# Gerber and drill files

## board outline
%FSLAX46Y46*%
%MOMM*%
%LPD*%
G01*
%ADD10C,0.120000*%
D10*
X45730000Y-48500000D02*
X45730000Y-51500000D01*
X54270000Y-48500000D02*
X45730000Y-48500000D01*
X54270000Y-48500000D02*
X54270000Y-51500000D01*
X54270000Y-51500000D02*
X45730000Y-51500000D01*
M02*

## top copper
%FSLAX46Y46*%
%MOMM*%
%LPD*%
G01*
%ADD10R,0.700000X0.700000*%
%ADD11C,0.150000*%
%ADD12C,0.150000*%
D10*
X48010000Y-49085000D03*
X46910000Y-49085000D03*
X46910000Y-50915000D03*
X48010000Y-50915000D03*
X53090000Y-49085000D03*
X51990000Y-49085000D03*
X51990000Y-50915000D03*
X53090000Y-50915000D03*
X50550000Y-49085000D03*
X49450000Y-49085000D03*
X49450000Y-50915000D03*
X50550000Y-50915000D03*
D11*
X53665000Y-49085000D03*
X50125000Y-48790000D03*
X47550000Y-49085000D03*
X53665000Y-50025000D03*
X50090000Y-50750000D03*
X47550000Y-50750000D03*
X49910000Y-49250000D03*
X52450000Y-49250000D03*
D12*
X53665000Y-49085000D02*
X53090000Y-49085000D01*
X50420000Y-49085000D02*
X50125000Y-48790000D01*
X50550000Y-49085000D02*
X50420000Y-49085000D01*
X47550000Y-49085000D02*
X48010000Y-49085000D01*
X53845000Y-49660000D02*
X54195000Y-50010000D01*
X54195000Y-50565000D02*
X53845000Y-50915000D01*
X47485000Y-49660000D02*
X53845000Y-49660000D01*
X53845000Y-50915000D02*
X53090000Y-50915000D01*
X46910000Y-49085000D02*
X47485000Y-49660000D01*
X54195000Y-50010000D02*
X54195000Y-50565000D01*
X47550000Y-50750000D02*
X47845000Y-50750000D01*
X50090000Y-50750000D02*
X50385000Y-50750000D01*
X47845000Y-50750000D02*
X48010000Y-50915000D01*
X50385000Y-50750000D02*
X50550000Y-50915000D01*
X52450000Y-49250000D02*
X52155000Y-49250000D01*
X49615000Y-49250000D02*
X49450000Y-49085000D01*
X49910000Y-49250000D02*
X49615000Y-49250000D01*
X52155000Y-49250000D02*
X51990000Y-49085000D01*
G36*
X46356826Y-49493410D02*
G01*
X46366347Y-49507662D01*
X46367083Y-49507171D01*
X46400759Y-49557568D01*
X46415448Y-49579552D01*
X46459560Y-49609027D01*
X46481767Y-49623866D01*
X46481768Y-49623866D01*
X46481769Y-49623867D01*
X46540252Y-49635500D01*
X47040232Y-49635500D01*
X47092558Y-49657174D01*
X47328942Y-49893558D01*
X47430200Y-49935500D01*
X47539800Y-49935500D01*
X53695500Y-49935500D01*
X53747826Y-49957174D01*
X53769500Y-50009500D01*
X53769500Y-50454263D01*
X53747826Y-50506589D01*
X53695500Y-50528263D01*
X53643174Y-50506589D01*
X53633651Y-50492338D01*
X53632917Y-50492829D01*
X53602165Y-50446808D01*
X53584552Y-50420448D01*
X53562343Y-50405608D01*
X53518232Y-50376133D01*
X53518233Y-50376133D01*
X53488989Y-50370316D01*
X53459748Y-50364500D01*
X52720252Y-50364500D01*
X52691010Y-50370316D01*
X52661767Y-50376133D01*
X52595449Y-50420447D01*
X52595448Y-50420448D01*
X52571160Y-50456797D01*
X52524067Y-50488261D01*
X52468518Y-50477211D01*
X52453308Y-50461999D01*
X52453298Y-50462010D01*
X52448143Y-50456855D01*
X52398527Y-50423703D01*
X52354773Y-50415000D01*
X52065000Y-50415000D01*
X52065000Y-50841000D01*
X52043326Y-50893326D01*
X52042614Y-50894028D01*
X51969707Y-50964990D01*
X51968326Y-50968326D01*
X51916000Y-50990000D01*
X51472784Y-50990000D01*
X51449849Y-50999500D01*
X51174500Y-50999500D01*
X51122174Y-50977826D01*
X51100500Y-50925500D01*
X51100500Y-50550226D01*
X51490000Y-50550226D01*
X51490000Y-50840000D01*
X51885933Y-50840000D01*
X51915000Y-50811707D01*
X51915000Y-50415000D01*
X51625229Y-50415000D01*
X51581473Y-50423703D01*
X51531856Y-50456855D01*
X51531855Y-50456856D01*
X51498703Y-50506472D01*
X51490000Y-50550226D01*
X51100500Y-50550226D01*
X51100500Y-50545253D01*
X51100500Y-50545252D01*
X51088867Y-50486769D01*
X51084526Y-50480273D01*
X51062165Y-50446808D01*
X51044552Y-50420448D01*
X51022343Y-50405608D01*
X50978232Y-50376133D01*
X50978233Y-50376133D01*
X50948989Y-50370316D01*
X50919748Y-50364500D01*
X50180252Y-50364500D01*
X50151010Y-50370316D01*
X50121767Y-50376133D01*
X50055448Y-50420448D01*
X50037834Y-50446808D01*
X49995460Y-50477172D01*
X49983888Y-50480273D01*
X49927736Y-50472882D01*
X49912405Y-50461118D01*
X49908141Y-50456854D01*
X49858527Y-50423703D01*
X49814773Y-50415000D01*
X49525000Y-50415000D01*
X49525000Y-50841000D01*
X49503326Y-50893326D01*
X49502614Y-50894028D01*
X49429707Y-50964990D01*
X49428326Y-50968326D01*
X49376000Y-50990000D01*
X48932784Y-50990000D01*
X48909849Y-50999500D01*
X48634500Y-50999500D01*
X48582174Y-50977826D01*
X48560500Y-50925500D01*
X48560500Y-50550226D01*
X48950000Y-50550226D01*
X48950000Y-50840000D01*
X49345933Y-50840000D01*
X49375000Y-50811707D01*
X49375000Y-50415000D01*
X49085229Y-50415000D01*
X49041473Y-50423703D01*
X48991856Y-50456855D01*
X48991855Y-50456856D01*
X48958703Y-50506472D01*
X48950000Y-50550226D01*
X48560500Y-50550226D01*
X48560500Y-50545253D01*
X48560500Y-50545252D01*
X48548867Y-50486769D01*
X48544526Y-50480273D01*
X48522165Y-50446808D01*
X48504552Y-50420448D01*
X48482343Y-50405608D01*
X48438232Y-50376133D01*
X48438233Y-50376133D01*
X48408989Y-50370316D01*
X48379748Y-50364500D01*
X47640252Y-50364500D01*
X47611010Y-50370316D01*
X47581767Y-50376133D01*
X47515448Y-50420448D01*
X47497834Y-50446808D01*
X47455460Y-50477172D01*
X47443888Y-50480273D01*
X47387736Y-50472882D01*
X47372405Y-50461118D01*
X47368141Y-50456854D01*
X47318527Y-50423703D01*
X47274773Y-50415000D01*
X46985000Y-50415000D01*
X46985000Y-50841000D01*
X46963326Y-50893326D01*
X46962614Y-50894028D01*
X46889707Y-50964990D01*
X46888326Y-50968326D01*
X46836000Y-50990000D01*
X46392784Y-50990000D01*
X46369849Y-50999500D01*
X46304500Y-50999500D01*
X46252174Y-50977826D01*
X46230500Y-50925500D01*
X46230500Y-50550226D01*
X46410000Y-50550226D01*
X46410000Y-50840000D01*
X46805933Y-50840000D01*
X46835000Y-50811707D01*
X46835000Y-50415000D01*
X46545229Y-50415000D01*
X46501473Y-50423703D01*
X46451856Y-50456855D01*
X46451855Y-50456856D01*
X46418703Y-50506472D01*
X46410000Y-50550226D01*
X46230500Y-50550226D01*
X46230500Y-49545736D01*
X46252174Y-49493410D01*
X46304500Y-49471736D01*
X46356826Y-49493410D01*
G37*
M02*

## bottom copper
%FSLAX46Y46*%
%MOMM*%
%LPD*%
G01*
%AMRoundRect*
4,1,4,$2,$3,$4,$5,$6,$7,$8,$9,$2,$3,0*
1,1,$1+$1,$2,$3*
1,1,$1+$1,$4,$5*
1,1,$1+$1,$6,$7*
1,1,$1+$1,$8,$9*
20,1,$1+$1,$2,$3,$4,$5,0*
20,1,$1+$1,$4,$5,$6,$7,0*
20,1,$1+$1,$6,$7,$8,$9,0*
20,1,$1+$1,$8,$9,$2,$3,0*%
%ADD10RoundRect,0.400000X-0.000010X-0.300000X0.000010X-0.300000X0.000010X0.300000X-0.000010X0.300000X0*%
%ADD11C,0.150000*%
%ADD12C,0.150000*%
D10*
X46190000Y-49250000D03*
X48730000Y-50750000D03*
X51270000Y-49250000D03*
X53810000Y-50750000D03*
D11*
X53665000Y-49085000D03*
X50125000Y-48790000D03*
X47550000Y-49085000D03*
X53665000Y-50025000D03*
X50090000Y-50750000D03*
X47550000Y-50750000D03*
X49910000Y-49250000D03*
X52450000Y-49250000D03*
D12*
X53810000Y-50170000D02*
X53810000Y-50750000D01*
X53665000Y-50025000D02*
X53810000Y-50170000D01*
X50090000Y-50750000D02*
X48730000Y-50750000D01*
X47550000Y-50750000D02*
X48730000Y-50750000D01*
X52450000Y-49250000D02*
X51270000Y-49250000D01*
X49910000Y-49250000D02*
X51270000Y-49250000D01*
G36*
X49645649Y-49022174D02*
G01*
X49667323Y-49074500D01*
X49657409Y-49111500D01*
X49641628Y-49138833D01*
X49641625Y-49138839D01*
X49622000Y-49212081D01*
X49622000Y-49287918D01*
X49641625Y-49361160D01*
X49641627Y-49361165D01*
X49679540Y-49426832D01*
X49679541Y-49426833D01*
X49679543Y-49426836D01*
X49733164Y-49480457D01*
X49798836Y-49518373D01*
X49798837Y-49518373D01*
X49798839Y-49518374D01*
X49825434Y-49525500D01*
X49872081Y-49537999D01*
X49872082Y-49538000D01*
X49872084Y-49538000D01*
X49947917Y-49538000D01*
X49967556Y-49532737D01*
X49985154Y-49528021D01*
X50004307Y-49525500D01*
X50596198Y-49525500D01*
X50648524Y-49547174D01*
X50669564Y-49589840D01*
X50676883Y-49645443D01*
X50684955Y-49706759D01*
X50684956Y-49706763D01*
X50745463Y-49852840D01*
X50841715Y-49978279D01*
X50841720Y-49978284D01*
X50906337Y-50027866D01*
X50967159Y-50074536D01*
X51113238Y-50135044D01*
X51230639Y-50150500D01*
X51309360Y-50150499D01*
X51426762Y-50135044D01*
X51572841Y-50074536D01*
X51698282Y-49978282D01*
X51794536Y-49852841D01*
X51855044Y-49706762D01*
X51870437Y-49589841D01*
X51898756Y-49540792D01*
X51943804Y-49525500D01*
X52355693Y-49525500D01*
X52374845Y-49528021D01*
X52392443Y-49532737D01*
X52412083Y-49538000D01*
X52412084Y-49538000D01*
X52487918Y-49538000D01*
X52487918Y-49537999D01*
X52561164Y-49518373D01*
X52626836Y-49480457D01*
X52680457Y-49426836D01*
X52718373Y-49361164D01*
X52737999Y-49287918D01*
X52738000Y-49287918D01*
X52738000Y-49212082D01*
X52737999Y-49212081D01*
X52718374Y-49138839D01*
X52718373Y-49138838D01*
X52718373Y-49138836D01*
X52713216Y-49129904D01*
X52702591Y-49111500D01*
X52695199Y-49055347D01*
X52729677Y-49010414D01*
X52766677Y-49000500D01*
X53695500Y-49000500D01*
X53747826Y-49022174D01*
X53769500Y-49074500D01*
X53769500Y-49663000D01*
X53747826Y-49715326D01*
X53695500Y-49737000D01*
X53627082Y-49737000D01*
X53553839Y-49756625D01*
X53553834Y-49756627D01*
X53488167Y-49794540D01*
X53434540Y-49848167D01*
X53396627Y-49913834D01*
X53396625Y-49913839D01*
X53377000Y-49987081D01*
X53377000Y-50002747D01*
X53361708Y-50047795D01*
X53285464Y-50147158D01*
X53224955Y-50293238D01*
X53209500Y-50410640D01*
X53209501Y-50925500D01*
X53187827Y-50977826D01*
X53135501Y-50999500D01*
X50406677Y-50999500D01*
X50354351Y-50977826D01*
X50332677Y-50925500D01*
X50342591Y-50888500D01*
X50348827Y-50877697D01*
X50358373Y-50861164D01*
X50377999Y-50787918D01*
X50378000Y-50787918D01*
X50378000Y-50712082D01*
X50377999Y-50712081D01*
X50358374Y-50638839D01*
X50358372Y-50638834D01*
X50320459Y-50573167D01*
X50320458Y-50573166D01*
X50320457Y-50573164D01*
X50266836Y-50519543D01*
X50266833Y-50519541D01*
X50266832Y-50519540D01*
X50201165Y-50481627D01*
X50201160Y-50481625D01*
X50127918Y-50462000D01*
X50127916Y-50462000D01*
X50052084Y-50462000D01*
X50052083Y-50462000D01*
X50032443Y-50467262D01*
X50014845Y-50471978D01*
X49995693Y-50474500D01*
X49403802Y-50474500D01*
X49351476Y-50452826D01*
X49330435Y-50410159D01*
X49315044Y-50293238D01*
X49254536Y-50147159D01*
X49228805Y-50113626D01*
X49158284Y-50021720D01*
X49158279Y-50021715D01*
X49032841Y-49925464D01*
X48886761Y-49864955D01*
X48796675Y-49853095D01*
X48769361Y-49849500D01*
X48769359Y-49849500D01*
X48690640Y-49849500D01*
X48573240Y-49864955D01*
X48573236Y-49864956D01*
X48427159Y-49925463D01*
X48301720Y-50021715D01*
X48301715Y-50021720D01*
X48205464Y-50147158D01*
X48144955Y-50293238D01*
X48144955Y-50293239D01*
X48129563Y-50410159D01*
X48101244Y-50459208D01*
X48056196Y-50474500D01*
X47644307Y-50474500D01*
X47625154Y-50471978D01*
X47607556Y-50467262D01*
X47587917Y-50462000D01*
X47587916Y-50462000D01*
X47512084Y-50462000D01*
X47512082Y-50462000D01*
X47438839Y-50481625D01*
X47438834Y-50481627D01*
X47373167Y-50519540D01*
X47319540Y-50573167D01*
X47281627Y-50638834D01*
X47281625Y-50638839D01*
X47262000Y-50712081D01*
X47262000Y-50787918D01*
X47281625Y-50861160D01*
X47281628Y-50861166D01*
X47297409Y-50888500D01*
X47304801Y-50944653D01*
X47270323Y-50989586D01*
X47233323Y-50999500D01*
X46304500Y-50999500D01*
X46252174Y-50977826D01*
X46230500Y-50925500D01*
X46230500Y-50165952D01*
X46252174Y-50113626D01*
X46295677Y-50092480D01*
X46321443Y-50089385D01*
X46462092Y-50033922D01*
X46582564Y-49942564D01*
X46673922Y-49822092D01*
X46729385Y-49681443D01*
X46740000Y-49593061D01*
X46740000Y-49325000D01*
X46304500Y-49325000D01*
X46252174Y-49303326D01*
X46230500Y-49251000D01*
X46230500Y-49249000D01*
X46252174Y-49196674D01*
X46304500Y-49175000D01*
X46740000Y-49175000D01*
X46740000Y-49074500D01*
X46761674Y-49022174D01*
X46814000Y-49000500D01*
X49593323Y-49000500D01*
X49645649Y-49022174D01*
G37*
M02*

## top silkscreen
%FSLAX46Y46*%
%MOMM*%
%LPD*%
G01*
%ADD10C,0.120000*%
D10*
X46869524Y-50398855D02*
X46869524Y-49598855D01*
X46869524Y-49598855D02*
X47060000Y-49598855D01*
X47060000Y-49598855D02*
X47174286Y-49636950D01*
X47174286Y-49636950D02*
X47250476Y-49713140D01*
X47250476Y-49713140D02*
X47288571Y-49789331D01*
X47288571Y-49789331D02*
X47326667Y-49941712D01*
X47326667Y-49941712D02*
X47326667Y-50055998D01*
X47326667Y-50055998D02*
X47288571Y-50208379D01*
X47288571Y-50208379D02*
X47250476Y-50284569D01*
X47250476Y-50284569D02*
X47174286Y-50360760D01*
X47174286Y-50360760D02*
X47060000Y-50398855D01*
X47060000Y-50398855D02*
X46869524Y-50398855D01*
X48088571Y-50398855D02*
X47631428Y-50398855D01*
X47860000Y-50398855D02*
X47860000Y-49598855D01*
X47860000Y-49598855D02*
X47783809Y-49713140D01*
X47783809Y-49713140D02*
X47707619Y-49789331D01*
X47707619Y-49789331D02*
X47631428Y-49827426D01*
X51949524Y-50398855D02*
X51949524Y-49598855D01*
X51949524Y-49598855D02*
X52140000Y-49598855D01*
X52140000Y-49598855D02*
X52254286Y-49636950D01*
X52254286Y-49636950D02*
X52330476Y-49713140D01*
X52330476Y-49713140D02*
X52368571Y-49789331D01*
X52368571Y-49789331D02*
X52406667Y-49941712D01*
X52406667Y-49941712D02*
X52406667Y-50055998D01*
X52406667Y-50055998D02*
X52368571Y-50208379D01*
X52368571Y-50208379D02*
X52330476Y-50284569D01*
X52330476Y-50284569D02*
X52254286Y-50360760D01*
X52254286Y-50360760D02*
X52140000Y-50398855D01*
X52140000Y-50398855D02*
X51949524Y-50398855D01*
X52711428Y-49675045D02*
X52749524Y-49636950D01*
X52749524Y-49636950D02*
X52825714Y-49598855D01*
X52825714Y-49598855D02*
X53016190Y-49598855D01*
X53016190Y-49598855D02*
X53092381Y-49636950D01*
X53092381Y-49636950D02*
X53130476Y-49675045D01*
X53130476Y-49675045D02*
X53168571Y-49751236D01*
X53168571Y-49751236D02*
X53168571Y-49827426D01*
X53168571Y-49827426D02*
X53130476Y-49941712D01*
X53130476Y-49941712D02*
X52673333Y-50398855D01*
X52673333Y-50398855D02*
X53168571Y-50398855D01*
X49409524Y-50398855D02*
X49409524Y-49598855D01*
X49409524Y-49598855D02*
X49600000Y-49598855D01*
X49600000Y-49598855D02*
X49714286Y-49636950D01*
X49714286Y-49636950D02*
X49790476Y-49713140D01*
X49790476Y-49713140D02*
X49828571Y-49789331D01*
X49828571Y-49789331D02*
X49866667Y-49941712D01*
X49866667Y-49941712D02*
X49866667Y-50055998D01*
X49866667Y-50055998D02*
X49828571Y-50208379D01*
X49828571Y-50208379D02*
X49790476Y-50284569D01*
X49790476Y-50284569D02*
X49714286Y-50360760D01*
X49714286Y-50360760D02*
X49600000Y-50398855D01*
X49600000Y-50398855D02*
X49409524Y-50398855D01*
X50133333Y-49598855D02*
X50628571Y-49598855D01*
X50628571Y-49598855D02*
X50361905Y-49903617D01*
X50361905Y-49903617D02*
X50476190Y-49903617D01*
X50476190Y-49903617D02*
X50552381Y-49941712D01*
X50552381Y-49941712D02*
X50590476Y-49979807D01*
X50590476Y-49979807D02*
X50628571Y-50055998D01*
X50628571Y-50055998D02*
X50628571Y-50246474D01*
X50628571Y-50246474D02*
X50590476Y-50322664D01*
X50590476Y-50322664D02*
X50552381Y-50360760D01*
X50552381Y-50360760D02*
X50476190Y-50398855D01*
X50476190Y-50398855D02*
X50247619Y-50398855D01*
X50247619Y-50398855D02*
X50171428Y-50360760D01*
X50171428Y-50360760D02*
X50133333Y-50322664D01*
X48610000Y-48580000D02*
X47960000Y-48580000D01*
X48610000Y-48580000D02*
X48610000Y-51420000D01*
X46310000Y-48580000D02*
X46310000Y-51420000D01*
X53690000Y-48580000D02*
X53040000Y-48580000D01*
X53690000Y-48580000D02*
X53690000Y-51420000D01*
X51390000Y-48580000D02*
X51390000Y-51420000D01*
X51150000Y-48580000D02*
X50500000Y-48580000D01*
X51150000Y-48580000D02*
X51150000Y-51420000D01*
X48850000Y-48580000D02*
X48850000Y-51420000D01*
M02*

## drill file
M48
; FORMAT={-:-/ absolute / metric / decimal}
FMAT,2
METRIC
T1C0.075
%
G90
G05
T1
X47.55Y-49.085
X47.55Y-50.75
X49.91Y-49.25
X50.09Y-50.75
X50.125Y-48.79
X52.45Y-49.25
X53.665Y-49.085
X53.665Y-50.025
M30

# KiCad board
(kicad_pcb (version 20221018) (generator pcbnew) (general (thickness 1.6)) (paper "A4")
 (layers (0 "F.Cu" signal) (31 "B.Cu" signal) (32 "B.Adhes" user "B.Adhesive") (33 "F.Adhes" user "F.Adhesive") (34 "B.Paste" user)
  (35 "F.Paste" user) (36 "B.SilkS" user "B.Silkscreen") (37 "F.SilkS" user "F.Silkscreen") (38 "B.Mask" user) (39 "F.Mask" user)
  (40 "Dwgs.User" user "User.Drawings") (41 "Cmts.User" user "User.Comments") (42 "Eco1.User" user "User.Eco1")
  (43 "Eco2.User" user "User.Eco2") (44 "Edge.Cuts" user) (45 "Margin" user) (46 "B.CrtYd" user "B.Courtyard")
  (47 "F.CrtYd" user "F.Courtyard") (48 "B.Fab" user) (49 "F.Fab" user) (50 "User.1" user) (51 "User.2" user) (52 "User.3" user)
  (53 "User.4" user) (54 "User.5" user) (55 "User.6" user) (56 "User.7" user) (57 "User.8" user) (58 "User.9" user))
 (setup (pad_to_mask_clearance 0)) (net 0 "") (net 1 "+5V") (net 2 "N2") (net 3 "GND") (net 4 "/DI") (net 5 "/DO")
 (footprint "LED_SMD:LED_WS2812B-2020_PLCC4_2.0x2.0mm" (layer "F.Cu") (at 47.46 50 -90)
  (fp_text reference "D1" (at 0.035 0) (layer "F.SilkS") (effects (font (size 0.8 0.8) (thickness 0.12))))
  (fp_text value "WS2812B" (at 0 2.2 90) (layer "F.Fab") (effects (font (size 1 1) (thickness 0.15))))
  (fp_line (start -1.42 -1.15) (end -1.42 -0.5) (stroke (width 0.12) (type solid)) (layer "F.SilkS"))
  (fp_line (start -1.42 -1.15) (end 1.42 -1.15) (stroke (width 0.12) (type solid)) (layer "F.SilkS"))
  (fp_line (start -1.42 1.15) (end 1.42 1.15) (stroke (width 0.12) (type solid)) (layer "F.SilkS"))
  (pad "1" smd rect (at -0.915 -0.55 270) (size 0.7 0.7) (layers "F.Cu" "F.Paste" "F.Mask") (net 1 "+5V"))
  (pad "2" smd rect (at -0.915 0.55 270) (size 0.7 0.7) (layers "F.Cu" "F.Paste" "F.Mask") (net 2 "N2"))
  (pad "3" smd rect (at 0.915 0.55 270) (size 0.7 0.7) (layers "F.Cu" "F.Paste" "F.Mask") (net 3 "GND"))
  (pad "4" smd rect (at 0.915 -0.55 270) (size 0.7 0.7) (layers "F.Cu" "F.Paste" "F.Mask") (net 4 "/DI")))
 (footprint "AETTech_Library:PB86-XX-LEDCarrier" (layer "F.Cu") (at 50 50)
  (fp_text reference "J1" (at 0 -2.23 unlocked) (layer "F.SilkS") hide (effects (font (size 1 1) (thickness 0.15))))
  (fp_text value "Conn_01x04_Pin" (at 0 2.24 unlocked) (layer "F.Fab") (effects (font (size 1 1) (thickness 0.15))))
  (fp_line (start -4.27 -1.5) (end -4.27 1.5) (stroke (width 0.12) (type default)) (layer "Edge.Cuts"))
  (fp_line (start 4.27 -1.5) (end -4.27 -1.5) (stroke (width 0.12) (type default)) (layer "Edge.Cuts"))
  (fp_line (start 4.27 -1.5) (end 4.27 1.5) (stroke (width 0.12) (type default)) (layer "Edge.Cuts"))
  (fp_line (start 4.27 1.5) (end -4.27 1.5) (stroke (width 0.12) (type default)) (layer "Edge.Cuts"))
  (pad "1" smd roundrect (at -3.81 -0.75) (size 0.8 1.4) (layers "B.Cu" "B.Paste" "B.Mask") (roundrect_rratio 0.5) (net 1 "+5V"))
  (pad "2" smd roundrect (at -1.27 0.75) (size 0.8 1.4) (layers "B.Cu" "B.Paste" "B.Mask") (roundrect_rratio 0.5) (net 4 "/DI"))
  (pad "3" smd roundrect (at 1.27 -0.75) (size 0.8 1.4) (layers "B.Cu" "B.Paste" "B.Mask") (roundrect_rratio 0.5) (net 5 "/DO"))
  (pad "4" smd roundrect (at 3.81 0.75) (size 0.8 1.4) (layers "B.Cu" "B.Paste" "B.Mask") (roundrect_rratio 0.5) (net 3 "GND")))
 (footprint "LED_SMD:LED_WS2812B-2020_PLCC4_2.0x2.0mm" (layer "F.Cu") (at 52.54 50 -90)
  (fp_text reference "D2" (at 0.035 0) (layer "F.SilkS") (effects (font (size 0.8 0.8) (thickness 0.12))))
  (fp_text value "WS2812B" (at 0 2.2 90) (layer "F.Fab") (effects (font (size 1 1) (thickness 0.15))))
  (fp_line (start -1.42 -1.15) (end -1.42 -0.5) (stroke (width 0.12) (type solid)) (layer "F.SilkS"))
  (fp_line (start -1.42 -1.15) (end 1.42 -1.15) (stroke (width 0.12) (type solid)) (layer "F.SilkS"))
  (fp_line (start -1.42 1.15) (end 1.42 1.15) (stroke (width 0.12) (type solid)) (layer "F.SilkS"))
  (pad "1" smd rect (at -0.915 -0.55 270) (size 0.7 0.7) (layers "F.Cu" "F.Paste" "F.Mask") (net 1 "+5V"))
  (pad "2" smd rect (at -0.915 0.55 270) (size 0.7 0.7) (layers "F.Cu" "F.Paste" "F.Mask") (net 5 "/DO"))
  (pad "3" smd rect (at 0.915 0.55 270) (size 0.7 0.7) (layers "F.Cu" "F.Paste" "F.Mask") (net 3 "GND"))
  (pad "4" smd rect (at 0.915 -0.55 270) (size 0.7 0.7) (layers "F.Cu" "F.Paste" "F.Mask") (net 2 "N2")))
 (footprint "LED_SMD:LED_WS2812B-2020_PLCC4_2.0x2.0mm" (layer "F.Cu") (at 50 50 -90)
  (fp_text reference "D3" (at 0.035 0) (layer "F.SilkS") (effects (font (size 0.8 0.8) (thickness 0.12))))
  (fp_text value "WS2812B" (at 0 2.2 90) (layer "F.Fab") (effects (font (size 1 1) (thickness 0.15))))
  (fp_line (start -1.42 -1.15) (end -1.42 -0.5) (stroke (width 0.12) (type solid)) (layer "F.SilkS"))
  (fp_line (start -1.42 -1.15) (end 1.42 -1.15) (stroke (width 0.12) (type solid)) (layer "F.SilkS"))
  (fp_line (start -1.42 1.15) (end 1.42 1.15) (stroke (width 0.12) (type solid)) (layer "F.SilkS"))
  (pad "1" smd rect (at -0.915 -0.55 270) (size 0.7 0.7) (layers "F.Cu" "F.Paste" "F.Mask") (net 1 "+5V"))
  (pad "2" smd rect (at -0.915 0.55 270) (size 0.7 0.7) (layers "F.Cu" "F.Paste" "F.Mask") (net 5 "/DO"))
  (pad "3" smd rect (at 0.915 0.55 270) (size 0.7 0.7) (layers "F.Cu" "F.Paste" "F.Mask") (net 3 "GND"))
  (pad "4" smd rect (at 0.915 -0.55 270) (size 0.7 0.7) (layers "F.Cu" "F.Paste" "F.Mask") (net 4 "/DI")))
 (segment (start 53.665 49.085) (end 53.09 49.085) (width 0.15) (layer "F.Cu") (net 1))
 (segment (start 50.42 49.085) (end 50.125 48.79) (width 0.15) (layer "F.Cu") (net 1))
 (segment (start 50.55 49.085) (end 50.42 49.085) (width 0.15) (layer "F.Cu") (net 1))
 (segment (start 47.55 49.085) (end 48.01 49.085) (width 0.15) (layer "F.Cu") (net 1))
 (via (at 53.665 49.085) (size 0.15) (drill 0.075) (layers "F.Cu" "B.Cu") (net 1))
 (via (at 50.125 48.79) (size 0.15) (drill 0.075) (layers "F.Cu" "B.Cu") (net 1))
 (via (at 47.55 49.085) (size 0.15) (drill 0.075) (layers "F.Cu" "B.Cu") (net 1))
 (segment (start 53.845 49.66) (end 54.195 50.01) (width 0.15) (layer "F.Cu") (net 2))
 (segment (start 54.195 50.565) (end 53.845 50.915) (width 0.15) (layer "F.Cu") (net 2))
 (segment (start 47.485 49.66) (end 53.845 49.66) (width 0.15) (layer "F.Cu") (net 2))
 (segment (start 53.845 50.915) (end 53.09 50.915) (width 0.15) (layer "F.Cu") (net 2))
 (segment (start 46.91 49.085) (end 47.485 49.66) (width 0.15) (layer "F.Cu") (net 2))
 (segment (start 54.195 50.01) (end 54.195 50.565) (width 0.15) (layer "F.Cu") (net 2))
 (via (at 53.665 50.025) (size 0.15) (drill 0.075) (layers "F.Cu" "B.Cu") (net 3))
 (segment (start 53.81 50.17) (end 53.81 50.75) (width 0.15) (layer "B.Cu") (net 3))
 (segment (start 53.665 50.025) (end 53.81 50.17) (width 0.15) (layer "B.Cu") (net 3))
 (segment (start 47.55 50.75) (end 47.845 50.75) (width 0.15) (layer "F.Cu") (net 4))
 (segment (start 50.09 50.75) (end 50.385 50.75) (width 0.15) (layer "F.Cu") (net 4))
 (segment (start 47.845 50.75) (end 48.01 50.915) (width 0.15) (layer "F.Cu") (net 4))
 (segment (start 50.385 50.75) (end 50.55 50.915) (width 0.15) (layer "F.Cu") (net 4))
 (via (at 50.09 50.75) (size 0.15) (drill 0.075) (layers "F.Cu" "B.Cu") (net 4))
 (via (at 47.55 50.75) (size 0.15) (drill 0.075) (layers "F.Cu" "B.Cu") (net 4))
 (segment (start 50.09 50.75) (end 48.73 50.75) (width 0.15) (layer "B.Cu") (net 4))
 (segment (start 47.55 50.75) (end 48.73 50.75) (width 0.15) (layer "B.Cu") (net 4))
 (segment (start 52.45 49.25) (end 52.155 49.25) (width 0.15) (layer "F.Cu") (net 5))
 (segment (start 49.615 49.25) (end 49.45 49.085) (width 0.15) (layer "F.Cu") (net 5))
 (segment (start 49.91 49.25) (end 49.615 49.25) (width 0.15) (layer "F.Cu") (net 5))
 (segment (start 52.155 49.25) (end 51.99 49.085) (width 0.15) (layer "F.Cu") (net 5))
 (via (at 49.91 49.25) (size 0.15) (drill 0.075) (layers "F.Cu" "B.Cu") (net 5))
 (via (at 52.45 49.25) (size 0.15) (drill 0.075) (layers "F.Cu" "B.Cu") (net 5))
 (segment (start 52.45 49.25) (end 51.27 49.25) (width 0.15) (layer "B.Cu") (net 5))
 (segment (start 49.91 49.25) (end 51.27 49.25) (width 0.15) (layer "B.Cu") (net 5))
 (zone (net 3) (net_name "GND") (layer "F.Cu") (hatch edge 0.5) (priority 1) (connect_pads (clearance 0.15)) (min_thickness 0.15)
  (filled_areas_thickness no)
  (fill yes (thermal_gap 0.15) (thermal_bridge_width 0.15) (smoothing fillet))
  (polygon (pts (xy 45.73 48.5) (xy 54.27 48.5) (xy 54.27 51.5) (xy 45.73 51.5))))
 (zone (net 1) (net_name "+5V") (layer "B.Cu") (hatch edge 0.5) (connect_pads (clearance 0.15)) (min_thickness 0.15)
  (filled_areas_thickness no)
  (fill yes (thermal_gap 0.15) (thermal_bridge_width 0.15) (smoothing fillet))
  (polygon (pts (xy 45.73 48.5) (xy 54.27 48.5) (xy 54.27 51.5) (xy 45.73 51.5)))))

